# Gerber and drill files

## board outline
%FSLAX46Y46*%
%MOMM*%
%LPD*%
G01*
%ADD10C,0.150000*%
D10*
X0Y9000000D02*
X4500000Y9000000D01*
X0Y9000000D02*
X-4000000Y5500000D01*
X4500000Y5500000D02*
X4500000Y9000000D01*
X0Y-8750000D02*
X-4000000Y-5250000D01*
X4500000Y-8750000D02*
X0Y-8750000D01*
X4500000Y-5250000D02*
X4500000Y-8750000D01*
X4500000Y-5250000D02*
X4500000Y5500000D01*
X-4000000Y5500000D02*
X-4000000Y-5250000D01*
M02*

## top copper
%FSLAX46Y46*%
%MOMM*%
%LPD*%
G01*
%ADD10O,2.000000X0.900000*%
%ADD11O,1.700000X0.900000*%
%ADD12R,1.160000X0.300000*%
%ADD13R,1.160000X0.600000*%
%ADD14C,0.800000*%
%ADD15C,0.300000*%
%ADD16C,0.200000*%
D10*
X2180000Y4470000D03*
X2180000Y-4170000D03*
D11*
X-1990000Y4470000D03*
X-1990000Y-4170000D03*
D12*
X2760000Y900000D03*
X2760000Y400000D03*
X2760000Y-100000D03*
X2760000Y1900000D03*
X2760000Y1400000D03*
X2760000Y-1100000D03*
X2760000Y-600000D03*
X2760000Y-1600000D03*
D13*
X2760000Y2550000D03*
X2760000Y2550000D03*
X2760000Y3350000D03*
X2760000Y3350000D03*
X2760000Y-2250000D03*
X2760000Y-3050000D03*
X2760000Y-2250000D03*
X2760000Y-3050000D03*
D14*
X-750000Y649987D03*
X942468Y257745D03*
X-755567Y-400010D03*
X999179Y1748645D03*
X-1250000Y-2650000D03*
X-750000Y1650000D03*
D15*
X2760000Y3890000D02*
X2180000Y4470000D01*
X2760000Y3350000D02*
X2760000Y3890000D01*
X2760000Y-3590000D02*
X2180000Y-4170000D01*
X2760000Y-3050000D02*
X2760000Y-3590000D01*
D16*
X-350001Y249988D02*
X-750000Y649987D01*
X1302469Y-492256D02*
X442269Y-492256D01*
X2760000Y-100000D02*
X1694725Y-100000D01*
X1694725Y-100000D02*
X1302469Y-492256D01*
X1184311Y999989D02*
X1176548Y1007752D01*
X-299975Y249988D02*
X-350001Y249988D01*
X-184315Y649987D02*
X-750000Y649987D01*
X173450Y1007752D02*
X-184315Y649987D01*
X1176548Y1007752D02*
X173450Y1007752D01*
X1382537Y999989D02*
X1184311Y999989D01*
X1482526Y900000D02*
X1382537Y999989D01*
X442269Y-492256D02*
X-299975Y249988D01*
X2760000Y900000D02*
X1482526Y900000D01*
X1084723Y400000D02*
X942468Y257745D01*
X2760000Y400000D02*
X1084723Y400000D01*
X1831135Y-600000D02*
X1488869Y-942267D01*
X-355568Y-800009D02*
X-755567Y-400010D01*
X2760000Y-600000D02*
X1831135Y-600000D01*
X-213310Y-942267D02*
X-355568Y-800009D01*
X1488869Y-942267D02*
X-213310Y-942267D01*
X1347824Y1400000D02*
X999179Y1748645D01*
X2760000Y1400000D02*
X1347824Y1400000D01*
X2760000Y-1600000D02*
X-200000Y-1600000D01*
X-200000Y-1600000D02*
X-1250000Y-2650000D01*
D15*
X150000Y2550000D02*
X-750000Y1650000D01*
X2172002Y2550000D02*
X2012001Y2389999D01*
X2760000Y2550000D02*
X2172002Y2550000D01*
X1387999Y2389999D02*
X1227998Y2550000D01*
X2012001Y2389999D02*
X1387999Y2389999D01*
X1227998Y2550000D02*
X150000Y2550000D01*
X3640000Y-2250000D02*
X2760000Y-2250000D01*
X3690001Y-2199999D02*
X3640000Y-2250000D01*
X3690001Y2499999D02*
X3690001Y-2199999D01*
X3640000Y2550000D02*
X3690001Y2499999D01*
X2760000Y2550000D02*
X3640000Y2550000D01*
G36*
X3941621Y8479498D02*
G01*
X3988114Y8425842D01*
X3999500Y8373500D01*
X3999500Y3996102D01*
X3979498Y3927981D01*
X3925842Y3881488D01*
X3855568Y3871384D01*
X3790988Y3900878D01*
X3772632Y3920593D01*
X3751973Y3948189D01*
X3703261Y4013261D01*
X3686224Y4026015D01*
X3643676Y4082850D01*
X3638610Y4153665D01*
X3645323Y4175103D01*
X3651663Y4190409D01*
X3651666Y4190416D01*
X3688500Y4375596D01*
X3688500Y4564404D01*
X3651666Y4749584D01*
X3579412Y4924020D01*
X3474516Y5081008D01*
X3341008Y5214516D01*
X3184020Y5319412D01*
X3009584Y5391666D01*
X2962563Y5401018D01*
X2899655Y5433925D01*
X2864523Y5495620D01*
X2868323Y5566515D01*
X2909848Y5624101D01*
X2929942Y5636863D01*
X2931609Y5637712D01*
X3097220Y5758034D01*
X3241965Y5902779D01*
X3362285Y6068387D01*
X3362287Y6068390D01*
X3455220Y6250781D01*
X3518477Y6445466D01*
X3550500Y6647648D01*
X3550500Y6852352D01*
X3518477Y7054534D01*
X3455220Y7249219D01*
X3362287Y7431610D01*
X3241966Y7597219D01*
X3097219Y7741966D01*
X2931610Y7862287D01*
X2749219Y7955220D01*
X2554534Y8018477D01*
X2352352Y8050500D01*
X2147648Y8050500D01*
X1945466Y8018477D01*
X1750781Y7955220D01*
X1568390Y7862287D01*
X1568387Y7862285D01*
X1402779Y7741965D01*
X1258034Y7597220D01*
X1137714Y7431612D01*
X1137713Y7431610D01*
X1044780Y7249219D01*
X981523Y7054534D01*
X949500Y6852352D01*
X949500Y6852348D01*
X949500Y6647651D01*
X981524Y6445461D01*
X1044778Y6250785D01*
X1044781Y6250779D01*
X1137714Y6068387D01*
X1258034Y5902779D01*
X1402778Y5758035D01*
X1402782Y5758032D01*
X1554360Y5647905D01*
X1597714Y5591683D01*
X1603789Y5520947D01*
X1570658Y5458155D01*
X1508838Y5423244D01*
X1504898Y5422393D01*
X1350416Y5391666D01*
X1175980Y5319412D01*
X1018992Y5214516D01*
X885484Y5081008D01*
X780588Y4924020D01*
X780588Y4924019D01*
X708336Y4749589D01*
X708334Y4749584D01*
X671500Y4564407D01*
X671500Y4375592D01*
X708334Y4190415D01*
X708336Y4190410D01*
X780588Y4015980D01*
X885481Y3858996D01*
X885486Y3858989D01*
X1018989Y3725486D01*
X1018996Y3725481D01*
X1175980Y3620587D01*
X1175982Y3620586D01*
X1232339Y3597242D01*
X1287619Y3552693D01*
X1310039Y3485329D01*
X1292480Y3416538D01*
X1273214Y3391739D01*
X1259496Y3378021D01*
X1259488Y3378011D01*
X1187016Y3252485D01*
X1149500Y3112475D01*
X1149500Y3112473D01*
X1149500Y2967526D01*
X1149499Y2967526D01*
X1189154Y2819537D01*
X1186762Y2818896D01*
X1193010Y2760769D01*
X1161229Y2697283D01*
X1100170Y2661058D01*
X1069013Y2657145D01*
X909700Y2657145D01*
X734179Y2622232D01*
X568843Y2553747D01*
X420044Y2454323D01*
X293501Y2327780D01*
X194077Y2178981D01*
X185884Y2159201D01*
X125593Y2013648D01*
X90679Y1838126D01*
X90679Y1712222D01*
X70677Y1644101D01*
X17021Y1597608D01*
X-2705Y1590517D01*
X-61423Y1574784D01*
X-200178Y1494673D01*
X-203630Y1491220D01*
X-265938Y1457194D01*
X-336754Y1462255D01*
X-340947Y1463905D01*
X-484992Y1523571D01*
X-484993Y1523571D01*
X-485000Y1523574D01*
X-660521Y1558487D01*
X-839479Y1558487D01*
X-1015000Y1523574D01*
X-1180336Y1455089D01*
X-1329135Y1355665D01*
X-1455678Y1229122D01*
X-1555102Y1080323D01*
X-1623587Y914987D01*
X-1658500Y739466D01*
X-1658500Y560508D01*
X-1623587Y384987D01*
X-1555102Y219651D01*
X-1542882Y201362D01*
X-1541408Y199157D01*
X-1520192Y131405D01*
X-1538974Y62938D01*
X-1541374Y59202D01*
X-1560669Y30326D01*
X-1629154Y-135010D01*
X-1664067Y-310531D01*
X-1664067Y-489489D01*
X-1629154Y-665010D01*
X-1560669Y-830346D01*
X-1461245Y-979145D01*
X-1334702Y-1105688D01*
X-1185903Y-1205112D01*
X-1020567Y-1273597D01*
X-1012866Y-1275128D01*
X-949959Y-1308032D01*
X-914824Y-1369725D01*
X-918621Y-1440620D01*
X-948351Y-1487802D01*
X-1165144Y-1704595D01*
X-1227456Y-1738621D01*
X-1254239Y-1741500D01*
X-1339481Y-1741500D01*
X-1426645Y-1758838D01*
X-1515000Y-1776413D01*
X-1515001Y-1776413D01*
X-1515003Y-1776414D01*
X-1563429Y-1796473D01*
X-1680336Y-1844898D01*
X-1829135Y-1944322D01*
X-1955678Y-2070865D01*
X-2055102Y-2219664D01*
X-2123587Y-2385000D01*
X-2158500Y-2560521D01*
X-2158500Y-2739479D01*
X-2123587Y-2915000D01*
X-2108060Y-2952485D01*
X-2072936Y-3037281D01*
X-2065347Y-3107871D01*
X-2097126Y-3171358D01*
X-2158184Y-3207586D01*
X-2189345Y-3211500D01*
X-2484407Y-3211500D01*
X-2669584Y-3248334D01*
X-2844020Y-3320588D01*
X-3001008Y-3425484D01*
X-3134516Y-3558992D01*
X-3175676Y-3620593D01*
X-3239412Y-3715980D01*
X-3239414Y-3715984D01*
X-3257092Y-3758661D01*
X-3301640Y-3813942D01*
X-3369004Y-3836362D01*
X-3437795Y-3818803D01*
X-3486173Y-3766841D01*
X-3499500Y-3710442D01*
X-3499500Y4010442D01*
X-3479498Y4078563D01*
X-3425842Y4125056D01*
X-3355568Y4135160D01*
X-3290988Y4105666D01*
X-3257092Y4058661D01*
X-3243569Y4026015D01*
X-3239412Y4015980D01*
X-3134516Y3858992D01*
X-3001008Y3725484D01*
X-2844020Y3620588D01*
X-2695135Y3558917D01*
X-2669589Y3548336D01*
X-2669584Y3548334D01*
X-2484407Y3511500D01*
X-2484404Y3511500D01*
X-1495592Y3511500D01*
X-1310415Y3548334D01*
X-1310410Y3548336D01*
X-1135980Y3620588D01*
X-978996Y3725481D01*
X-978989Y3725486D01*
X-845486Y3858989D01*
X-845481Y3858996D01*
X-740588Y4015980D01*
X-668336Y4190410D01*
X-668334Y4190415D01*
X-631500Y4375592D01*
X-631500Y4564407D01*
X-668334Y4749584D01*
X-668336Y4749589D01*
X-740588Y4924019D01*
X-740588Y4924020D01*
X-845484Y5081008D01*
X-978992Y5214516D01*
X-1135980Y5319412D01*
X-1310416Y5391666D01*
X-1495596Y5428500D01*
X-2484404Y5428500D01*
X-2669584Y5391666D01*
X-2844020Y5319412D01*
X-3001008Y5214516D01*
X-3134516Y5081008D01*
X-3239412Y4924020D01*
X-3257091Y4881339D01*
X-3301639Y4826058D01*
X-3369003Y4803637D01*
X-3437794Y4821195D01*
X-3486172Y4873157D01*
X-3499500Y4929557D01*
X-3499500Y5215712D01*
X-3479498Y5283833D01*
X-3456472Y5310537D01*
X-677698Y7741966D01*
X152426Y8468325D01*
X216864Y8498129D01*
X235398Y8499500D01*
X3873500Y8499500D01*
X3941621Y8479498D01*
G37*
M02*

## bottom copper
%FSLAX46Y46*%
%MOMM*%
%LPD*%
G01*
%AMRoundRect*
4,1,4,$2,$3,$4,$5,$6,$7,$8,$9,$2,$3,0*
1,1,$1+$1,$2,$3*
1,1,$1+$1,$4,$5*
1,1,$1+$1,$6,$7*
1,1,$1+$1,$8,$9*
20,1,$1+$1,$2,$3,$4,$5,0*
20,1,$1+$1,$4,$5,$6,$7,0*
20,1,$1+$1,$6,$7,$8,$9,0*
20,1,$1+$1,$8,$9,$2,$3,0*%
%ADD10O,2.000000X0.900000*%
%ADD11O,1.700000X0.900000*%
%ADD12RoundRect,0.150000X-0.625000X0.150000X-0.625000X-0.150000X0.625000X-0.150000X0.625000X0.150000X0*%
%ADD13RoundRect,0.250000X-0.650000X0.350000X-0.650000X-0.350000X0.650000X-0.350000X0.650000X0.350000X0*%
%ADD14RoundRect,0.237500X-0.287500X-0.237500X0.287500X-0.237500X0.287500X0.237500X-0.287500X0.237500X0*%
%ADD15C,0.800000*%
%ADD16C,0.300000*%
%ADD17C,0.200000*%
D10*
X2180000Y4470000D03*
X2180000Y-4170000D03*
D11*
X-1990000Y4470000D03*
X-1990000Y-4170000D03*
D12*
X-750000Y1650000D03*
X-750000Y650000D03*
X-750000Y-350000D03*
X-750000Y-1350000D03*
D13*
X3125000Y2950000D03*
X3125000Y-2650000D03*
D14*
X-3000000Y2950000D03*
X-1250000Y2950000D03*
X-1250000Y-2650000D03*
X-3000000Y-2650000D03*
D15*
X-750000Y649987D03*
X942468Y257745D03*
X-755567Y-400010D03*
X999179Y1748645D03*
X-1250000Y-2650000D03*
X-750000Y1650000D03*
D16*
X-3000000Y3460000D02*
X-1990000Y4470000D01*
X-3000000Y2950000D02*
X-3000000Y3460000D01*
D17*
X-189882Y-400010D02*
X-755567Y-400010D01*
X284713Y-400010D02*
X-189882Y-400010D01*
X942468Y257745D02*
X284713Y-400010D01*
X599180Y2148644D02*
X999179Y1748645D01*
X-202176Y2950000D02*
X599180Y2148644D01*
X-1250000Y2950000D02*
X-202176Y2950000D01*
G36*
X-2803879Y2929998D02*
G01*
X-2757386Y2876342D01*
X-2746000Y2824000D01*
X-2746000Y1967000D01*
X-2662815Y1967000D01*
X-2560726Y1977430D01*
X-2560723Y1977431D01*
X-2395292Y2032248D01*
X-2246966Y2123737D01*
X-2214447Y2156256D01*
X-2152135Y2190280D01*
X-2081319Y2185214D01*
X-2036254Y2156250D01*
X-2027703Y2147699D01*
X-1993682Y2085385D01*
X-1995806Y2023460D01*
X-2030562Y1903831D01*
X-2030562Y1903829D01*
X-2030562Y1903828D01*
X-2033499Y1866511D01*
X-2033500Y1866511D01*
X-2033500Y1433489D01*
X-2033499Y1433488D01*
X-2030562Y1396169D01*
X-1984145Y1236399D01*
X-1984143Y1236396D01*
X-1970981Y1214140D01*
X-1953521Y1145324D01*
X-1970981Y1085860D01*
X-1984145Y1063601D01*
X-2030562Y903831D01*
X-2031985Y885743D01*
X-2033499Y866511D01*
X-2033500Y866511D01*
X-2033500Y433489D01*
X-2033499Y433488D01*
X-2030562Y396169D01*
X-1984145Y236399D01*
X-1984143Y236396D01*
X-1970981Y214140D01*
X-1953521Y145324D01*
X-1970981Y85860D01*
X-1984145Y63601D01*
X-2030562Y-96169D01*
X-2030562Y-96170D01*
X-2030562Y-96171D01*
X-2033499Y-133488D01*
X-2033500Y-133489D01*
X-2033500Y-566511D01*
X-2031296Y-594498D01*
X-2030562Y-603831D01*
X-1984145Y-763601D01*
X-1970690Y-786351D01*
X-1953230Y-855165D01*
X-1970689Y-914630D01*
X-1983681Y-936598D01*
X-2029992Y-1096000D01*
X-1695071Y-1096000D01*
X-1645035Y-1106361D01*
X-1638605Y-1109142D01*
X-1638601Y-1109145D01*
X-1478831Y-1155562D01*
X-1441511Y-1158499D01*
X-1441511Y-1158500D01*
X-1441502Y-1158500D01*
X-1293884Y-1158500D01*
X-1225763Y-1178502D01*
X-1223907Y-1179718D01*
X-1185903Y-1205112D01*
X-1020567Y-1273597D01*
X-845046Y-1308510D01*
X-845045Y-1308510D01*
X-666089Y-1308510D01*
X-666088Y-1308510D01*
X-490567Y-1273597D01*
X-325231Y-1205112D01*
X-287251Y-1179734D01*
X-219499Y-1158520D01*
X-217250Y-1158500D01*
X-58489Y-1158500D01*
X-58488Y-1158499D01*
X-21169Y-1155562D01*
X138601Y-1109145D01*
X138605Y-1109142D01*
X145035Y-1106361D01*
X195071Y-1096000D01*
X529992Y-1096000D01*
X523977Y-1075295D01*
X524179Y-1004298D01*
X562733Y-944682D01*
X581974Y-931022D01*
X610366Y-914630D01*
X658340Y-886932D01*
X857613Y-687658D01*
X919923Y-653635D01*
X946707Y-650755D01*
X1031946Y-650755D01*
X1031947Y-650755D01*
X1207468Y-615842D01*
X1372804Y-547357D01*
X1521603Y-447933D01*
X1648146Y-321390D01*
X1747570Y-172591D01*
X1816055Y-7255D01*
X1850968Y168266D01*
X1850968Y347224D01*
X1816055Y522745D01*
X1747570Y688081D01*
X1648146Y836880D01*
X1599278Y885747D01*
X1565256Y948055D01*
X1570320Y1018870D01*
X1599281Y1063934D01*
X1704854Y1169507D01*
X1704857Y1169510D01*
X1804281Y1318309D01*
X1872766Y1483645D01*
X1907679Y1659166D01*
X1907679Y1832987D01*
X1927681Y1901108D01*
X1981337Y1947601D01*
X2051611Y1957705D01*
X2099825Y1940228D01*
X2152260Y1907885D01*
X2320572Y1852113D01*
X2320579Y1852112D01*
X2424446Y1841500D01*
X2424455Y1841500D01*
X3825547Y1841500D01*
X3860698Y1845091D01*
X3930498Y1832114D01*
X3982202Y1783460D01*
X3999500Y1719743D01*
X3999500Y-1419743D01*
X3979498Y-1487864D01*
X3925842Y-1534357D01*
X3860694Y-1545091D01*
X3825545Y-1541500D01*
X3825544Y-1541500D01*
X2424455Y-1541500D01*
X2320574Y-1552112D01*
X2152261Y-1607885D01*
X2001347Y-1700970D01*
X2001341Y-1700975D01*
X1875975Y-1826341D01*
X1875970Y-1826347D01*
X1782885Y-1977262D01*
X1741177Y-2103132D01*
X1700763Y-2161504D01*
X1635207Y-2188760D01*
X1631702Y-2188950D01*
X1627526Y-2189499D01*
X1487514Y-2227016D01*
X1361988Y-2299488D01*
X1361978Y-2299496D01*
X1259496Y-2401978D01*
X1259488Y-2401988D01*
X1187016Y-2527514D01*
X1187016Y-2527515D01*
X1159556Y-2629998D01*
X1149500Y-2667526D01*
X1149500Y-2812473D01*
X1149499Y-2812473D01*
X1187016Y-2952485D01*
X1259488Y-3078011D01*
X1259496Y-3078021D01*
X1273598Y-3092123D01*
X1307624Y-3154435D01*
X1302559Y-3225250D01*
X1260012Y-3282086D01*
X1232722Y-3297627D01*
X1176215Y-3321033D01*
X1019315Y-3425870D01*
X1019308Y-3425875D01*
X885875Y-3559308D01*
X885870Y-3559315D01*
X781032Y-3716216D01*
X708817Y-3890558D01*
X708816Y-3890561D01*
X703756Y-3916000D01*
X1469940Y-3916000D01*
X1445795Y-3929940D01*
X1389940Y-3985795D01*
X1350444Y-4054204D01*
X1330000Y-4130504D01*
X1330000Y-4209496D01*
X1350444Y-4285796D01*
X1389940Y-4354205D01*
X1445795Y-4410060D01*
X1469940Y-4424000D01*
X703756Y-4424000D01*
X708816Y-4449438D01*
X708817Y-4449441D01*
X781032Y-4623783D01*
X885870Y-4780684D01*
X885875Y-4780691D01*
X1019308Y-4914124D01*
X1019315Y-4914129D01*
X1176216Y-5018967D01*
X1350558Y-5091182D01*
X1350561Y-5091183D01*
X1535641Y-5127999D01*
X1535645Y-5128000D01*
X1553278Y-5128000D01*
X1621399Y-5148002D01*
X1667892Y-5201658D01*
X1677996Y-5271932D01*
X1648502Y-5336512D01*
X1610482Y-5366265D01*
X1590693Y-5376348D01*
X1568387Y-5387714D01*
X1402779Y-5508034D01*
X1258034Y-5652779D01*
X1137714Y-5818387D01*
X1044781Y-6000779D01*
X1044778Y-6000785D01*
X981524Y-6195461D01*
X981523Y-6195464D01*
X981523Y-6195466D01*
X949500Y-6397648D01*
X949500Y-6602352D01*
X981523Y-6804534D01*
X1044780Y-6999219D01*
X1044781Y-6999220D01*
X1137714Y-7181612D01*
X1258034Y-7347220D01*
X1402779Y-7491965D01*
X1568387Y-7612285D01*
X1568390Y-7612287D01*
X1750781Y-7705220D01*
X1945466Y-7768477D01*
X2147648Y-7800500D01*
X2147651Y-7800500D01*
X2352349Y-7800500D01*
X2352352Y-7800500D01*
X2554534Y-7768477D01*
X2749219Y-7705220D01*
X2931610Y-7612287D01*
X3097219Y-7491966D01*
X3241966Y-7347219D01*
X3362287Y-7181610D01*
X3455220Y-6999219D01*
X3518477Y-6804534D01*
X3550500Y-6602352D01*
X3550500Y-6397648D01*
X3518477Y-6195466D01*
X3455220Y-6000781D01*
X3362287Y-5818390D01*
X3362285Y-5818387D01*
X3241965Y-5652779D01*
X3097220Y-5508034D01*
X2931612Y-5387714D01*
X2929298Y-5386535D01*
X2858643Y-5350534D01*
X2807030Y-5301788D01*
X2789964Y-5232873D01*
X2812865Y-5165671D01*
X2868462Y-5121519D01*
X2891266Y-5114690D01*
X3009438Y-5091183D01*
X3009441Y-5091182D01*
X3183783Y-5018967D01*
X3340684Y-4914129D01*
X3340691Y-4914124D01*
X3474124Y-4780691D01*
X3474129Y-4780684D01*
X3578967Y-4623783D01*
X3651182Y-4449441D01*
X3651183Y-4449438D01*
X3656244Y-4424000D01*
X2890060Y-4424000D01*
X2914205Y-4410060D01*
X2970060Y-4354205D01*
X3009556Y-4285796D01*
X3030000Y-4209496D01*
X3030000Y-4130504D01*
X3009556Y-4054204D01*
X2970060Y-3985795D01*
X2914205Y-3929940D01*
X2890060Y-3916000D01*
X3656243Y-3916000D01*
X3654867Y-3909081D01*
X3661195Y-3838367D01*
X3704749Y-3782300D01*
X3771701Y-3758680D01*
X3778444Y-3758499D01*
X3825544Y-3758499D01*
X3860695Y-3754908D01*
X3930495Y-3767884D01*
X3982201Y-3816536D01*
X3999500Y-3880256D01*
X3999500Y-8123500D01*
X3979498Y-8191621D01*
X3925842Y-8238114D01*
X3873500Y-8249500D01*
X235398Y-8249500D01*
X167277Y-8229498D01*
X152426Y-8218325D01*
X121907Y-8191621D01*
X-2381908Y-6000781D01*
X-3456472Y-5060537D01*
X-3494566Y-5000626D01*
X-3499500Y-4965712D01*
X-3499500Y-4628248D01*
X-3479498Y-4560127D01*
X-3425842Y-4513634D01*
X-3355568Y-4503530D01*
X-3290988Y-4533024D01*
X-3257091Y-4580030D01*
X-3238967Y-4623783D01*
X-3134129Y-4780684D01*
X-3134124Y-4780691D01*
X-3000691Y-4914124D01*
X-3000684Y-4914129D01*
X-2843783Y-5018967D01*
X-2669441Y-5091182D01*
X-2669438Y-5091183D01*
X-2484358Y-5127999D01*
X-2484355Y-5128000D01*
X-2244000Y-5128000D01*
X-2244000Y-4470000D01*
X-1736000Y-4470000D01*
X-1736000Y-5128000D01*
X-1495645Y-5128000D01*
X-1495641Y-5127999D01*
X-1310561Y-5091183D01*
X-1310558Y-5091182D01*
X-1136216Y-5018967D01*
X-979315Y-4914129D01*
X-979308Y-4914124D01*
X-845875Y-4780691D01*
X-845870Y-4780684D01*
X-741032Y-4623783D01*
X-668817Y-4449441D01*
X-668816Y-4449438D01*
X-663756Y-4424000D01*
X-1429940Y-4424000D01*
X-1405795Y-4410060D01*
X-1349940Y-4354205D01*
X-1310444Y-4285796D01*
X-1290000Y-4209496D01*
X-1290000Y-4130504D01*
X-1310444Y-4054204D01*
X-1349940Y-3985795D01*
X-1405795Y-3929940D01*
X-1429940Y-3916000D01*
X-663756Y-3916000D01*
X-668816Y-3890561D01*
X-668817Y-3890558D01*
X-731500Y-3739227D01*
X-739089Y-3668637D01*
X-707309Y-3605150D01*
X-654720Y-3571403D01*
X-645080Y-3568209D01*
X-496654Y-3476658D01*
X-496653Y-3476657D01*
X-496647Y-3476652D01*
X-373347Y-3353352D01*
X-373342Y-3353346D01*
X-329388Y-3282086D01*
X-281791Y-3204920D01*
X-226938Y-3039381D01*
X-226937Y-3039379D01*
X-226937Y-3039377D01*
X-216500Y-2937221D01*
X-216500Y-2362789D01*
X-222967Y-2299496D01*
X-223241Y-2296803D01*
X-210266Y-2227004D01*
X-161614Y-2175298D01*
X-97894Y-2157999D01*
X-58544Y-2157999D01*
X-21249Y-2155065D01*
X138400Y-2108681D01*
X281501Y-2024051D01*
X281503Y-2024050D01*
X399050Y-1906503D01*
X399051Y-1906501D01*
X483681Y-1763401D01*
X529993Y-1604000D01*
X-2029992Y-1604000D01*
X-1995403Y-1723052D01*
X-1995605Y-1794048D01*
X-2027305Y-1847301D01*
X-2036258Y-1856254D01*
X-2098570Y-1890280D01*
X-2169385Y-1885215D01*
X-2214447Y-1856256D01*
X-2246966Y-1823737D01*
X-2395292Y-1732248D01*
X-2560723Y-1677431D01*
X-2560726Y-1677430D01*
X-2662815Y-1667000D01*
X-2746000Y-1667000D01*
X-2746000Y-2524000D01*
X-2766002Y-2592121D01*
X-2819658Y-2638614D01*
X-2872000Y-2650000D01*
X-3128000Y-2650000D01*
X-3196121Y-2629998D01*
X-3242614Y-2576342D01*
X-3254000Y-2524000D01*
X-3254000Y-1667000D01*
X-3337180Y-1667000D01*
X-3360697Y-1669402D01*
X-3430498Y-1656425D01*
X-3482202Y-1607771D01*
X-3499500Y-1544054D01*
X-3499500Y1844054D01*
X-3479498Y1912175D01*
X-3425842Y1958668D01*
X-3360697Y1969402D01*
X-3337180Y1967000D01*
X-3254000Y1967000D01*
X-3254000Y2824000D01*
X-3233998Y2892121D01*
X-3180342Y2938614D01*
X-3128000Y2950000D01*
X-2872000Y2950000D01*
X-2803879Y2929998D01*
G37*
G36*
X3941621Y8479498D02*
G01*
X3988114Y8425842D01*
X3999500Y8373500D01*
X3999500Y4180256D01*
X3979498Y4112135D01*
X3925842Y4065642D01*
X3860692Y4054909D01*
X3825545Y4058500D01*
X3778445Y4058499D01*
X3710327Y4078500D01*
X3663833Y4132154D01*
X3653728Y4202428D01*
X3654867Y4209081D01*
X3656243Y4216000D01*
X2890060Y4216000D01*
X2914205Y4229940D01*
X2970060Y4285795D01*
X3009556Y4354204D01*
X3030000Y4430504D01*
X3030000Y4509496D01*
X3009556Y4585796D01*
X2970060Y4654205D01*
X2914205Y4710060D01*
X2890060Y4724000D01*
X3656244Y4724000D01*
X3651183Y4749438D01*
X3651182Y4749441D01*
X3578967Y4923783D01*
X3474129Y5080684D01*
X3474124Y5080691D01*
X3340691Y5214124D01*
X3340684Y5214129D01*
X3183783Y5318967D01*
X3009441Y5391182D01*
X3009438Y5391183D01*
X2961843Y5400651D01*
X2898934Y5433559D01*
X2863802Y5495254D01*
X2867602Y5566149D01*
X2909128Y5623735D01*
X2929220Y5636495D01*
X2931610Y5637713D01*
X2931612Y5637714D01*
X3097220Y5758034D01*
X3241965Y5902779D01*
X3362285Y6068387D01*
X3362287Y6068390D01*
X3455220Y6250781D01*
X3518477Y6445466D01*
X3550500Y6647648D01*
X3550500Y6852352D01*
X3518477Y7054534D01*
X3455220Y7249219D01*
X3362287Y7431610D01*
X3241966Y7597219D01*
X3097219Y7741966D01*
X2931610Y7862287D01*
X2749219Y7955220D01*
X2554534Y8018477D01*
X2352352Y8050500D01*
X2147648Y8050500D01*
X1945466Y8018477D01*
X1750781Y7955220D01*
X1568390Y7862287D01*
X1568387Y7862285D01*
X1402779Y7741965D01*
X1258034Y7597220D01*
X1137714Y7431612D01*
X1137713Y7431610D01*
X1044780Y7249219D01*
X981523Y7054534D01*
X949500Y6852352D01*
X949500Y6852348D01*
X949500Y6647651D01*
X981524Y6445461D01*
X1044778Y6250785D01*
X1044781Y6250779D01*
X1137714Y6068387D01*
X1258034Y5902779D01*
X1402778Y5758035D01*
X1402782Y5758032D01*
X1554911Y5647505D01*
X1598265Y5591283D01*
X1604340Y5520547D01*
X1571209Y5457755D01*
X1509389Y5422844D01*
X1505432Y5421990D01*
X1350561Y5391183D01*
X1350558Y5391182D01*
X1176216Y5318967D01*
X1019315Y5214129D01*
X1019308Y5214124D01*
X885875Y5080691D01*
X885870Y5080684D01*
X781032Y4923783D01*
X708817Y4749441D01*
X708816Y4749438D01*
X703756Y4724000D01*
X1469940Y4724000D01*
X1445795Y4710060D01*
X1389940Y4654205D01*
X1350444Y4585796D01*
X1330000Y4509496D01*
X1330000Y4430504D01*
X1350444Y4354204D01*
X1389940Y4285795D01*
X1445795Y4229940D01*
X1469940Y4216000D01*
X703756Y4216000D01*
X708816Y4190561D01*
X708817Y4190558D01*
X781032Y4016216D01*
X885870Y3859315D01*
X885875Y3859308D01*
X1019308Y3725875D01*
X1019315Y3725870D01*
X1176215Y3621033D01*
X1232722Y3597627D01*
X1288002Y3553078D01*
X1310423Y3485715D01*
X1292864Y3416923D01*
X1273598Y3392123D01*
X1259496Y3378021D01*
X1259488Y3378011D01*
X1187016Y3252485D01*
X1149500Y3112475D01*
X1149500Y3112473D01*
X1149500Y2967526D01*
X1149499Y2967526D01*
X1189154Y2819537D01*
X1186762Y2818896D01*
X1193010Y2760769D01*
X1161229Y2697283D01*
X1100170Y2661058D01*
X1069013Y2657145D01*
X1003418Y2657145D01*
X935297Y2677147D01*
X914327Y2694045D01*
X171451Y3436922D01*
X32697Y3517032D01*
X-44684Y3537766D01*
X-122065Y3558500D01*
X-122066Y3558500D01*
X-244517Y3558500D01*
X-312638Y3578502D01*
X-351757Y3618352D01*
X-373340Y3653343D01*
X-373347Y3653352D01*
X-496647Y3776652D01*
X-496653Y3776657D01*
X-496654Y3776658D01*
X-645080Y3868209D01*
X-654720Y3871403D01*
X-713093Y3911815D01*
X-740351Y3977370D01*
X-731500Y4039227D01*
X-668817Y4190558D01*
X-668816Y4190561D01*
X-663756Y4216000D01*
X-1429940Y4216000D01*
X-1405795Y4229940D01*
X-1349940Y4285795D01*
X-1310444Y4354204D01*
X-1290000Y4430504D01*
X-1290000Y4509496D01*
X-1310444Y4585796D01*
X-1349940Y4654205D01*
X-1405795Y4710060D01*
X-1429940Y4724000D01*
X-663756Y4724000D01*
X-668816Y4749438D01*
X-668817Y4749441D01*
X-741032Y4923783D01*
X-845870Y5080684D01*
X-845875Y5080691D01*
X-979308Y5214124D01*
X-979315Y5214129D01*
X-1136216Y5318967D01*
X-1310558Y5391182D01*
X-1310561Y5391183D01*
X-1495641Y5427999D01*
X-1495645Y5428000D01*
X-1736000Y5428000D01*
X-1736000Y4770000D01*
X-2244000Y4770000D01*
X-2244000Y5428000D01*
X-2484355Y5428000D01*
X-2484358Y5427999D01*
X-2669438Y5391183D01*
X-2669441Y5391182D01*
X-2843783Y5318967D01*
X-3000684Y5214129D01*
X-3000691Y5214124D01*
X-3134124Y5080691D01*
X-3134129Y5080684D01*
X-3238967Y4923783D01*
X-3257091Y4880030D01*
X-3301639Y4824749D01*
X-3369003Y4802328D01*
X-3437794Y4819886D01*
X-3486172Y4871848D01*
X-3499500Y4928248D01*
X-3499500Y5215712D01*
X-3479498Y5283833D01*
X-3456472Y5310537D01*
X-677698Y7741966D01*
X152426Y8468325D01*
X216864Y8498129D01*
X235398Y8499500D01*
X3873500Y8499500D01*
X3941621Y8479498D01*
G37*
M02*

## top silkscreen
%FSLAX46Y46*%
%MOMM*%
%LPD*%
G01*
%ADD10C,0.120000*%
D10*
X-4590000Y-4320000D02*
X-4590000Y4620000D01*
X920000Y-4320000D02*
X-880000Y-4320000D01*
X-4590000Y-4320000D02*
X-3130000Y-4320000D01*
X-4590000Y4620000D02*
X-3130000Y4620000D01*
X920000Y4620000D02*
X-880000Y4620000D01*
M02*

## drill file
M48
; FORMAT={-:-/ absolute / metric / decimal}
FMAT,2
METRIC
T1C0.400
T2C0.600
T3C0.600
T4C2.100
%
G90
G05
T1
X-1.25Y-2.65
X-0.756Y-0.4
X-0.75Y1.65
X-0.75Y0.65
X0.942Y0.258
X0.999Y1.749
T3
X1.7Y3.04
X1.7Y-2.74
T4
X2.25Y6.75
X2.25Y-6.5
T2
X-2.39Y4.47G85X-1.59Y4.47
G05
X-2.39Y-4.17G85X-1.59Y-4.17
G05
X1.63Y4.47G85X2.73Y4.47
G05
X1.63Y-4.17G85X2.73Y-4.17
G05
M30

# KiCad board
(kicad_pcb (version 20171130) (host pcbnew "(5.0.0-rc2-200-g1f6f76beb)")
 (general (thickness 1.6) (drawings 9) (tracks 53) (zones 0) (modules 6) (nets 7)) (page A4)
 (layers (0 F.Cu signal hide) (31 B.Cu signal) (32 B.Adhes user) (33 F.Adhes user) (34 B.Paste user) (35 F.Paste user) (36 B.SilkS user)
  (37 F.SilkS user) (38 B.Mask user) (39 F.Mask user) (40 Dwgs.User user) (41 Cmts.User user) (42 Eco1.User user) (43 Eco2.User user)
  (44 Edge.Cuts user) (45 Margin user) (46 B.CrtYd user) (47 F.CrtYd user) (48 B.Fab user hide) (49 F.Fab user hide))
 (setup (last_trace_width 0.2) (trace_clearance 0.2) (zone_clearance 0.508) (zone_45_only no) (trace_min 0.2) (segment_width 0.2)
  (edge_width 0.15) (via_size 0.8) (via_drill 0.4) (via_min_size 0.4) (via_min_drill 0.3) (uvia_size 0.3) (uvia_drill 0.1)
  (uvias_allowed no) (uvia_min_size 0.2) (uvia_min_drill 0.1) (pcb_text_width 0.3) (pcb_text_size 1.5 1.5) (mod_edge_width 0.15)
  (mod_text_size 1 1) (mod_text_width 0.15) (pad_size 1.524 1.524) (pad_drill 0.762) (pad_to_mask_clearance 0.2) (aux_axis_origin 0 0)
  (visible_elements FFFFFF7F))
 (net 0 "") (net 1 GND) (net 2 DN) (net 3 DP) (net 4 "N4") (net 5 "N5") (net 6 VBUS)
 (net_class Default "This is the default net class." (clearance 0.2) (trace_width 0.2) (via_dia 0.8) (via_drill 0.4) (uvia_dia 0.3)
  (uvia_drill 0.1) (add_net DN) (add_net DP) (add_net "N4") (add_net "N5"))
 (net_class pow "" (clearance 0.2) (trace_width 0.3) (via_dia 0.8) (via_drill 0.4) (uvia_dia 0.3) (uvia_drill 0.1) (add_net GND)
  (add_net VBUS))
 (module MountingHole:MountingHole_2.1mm (layer F.Cu) (at 2.25 -6.75)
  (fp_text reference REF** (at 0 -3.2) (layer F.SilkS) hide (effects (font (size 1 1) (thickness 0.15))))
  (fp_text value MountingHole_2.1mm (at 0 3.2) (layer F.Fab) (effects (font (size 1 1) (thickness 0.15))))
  (pad "" np_thru_hole circle (at 0 0) (size 2.1 2.1) (drill 2.1) (layers *.Cu *.Mask)))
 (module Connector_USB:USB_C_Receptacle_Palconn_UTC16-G (layer F.Cu) (at 0.25 -0.15 270)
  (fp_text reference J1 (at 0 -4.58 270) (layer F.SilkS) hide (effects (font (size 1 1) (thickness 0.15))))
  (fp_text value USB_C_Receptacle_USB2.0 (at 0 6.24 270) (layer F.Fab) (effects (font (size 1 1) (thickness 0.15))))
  (fp_line (start 4.47 4.84) (end -4.47 4.84) (layer F.SilkS) (width 0.12))
  (fp_line (start 4.47 -0.67) (end 4.47 1.13) (layer F.SilkS) (width 0.12))
  (fp_line (start 4.47 4.84) (end 4.47 3.38) (layer F.SilkS) (width 0.12))
  (fp_line (start -4.47 4.84) (end -4.47 3.38) (layer F.SilkS) (width 0.12))
  (fp_line (start -4.47 -0.67) (end -4.47 1.13) (layer F.SilkS) (width 0.12))
  (pad S1 thru_hole oval (at -4.32 -1.93) (size 2 0.9) (drill oval 1.7 0.6) (layers *.Cu *.Mask) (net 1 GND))
  (pad S1 thru_hole oval (at 4.32 -1.93) (size 2 0.9) (drill oval 1.7 0.6) (layers *.Cu *.Mask) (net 1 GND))
  (pad S1 thru_hole oval (at -4.32 2.24) (size 1.7 0.9) (drill oval 1.4 0.6) (layers *.Cu *.Mask) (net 1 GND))
  (pad S1 thru_hole oval (at 4.32 2.24) (size 1.7 0.9) (drill oval 1.4 0.6) (layers *.Cu *.Mask) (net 1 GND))
  (pad B7 smd rect (at -0.75 -2.51 90) (size 0.3 1.16) (layers F.Cu F.Paste F.Mask) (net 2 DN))
  (pad A6 smd rect (at -0.25 -2.51 90) (size 0.3 1.16) (layers F.Cu F.Paste F.Mask) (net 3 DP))
  (pad A7 smd rect (at 0.25 -2.51 90) (size 0.3 1.16) (layers F.Cu F.Paste F.Mask) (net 2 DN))
  (pad B8 smd rect (at -1.75 -2.51 90) (size 0.3 1.16) (layers F.Cu F.Paste F.Mask))
  (pad A5 smd rect (at -1.25 -2.51 90) (size 0.3 1.16) (layers F.Cu F.Paste F.Mask) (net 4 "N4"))
  (pad A8 smd rect (at 1.25 -2.51 90) (size 0.3 1.16) (layers F.Cu F.Paste F.Mask))
  (pad B6 smd rect (at 0.75 -2.51 90) (size 0.3 1.16) (layers F.Cu F.Paste F.Mask) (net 3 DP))
  (pad B5 smd rect (at 1.75 -2.51 90) (size 0.3 1.16) (layers F.Cu F.Paste F.Mask) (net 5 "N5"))
  (pad "" np_thru_hole circle (at 2.89 -1.45 90) (size 0.6 0.6) (drill 0.6) (layers *.Cu *.Mask))
  (pad "" np_thru_hole circle (at -2.89 -1.45 90) (size 0.6 0.6) (drill 0.6) (layers *.Cu *.Mask))
  (pad A4 smd rect (at -2.4 -2.51 270) (size 0.6 1.16) (layers F.Cu F.Paste F.Mask) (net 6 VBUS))
  (pad B9 smd rect (at -2.4 -2.51 270) (size 0.6 1.16) (layers F.Cu F.Paste F.Mask) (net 6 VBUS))
  (pad A1 smd rect (at -3.2 -2.51 270) (size 0.6 1.16) (layers F.Cu F.Paste F.Mask) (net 1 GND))
  (pad B12 smd rect (at -3.2 -2.51 270) (size 0.6 1.16) (layers F.Cu F.Paste F.Mask) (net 1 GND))
  (pad B4 smd rect (at 2.4 -2.51 270) (size 0.6 1.16) (layers F.Cu F.Paste F.Mask) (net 6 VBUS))
  (pad B1 smd rect (at 3.2 -2.51 270) (size 0.6 1.16) (layers F.Cu F.Paste F.Mask) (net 1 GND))
  (pad A9 smd rect (at 2.4 -2.51 270) (size 0.6 1.16) (layers F.Cu F.Paste F.Mask) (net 6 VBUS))
  (pad A12 smd rect (at 3.2 -2.51 270) (size 0.6 1.16) (layers F.Cu F.Paste F.Mask) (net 1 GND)))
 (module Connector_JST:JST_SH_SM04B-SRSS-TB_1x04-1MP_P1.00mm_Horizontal (layer B.Cu) (at 1.25 -0.15 270)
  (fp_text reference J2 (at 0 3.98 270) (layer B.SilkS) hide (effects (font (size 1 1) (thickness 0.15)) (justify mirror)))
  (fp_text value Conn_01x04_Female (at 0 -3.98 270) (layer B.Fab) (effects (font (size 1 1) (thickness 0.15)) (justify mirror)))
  (pad 1 smd roundrect (at -1.5 2 270) (size 0.6 1.55) (layers B.Cu B.Paste B.Mask) (roundrect_rratio 0.25) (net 6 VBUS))
  (pad 2 smd roundrect (at -0.5 2 270) (size 0.6 1.55) (layers B.Cu B.Paste B.Mask) (roundrect_rratio 0.25) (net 2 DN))
  (pad 3 smd roundrect (at 0.5 2 270) (size 0.6 1.55) (layers B.Cu B.Paste B.Mask) (roundrect_rratio 0.25) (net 3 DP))
  (pad 4 smd roundrect (at 1.5 2 270) (size 0.6 1.55) (layers B.Cu B.Paste B.Mask) (roundrect_rratio 0.25) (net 1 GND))
  (pad MP smd roundrect (at -2.8 -1.875 270) (size 1.2 1.8) (layers B.Cu B.Paste B.Mask) (roundrect_rratio 0.208333))
  (pad MP smd roundrect (at 2.8 -1.875 270) (size 1.2 1.8) (layers B.Cu B.Paste B.Mask) (roundrect_rratio 0.208333)))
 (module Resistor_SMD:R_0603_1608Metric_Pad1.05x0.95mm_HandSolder (layer B.Cu) (at -2.125 -2.95)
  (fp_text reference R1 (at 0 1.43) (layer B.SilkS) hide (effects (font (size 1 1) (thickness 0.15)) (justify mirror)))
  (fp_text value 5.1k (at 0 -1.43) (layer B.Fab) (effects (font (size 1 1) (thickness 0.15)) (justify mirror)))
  (pad 1 smd roundrect (at -0.875 0) (size 1.05 0.95) (layers B.Cu B.Paste B.Mask) (roundrect_rratio 0.25) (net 1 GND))
  (pad 2 smd roundrect (at 0.875 0) (size 1.05 0.95) (layers B.Cu B.Paste B.Mask) (roundrect_rratio 0.25) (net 4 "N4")))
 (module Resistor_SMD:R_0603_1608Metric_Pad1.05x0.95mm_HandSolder (layer B.Cu) (at -2.125 2.65)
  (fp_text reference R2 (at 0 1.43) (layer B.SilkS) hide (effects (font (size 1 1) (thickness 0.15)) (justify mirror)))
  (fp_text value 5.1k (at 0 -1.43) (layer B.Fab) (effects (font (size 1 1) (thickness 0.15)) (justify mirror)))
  (pad 2 smd roundrect (at 0.875 0) (size 1.05 0.95) (layers B.Cu B.Paste B.Mask) (roundrect_rratio 0.25) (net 5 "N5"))
  (pad 1 smd roundrect (at -0.875 0) (size 1.05 0.95) (layers B.Cu B.Paste B.Mask) (roundrect_rratio 0.25) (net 1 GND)))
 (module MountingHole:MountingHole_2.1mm (layer F.Cu) (at 2.25 6.5)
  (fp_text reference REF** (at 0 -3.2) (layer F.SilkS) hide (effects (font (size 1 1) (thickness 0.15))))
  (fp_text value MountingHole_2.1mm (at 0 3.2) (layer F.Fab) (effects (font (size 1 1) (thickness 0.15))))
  (pad "" np_thru_hole circle (at 0 0) (size 2.1 2.1) (drill 2.1) (layers *.Cu *.Mask)))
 (gr_line (start 0 -9) (end 4.5 -9) (layer Edge.Cuts) (width 0.15))
 (gr_line (start 0 -9) (end -4 -5.5) (layer Edge.Cuts) (width 0.15))
 (gr_line (start 4.5 -5.5) (end 4.5 -9) (layer Edge.Cuts) (width 0.15))
 (gr_line (start 0 8.75) (end -4 5.25) (layer Edge.Cuts) (width 0.15))
 (gr_line (start 4.5 8.75) (end 0 8.75) (layer Edge.Cuts) (width 0.15))
 (gr_line (start 4.5 5.25) (end 4.5 8.75) (layer Edge.Cuts) (width 0.15))
 (gr_line (start 4.5 5.25) (end 4.5 -5.5) (layer Edge.Cuts) (width 0.15))
 (gr_line (start -4 -5.5) (end -4 5.25) (layer Edge.Cuts) (width 0.15))
 (segment (start 2.76 -3.89) (end 2.18 -4.47) (width 0.3) (layer F.Cu) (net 1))
 (segment (start 2.76 -3.35) (end 2.76 -3.89) (width 0.3) (layer F.Cu) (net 1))
 (segment (start 2.76 3.59) (end 2.18 4.17) (width 0.3) (layer F.Cu) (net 1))
 (segment (start 2.76 3.05) (end 2.76 3.59) (width 0.3) (layer F.Cu) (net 1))
 (segment (start -3 -3.46) (end -1.99 -4.47) (width 0.3) (layer B.Cu) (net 1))
 (segment (start -3 -2.95) (end -3 -3.46) (width 0.3) (layer B.Cu) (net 1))
 (via (at -0.75 -0.649987) (size 0.8) (drill 0.4) (layers F.Cu B.Cu) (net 2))
 (segment (start -0.350001 -0.249988) (end -0.75 -0.649987) (width 0.2) (layer F.Cu) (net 2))
 (segment (start 1.302469 0.492256) (end 0.442269 0.492256) (width 0.2) (layer F.Cu) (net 2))
 (segment (start 2.76 0.1) (end 1.694725 0.1) (width 0.2) (layer F.Cu) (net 2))
 (segment (start 1.694725 0.1) (end 1.302469 0.492256) (width 0.2) (layer F.Cu) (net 2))
 (segment (start 1.184311 -0.999989) (end 1.176548 -1.007752) (width 0.2) (layer F.Cu) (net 2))
 (segment (start -0.299975 -0.249988) (end -0.350001 -0.249988) (width 0.2) (layer F.Cu) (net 2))
 (segment (start -0.184315 -0.649987) (end -0.75 -0.649987) (width 0.2) (layer F.Cu) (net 2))
 (segment (start 0.17345 -1.007752) (end -0.184315 -0.649987) (width 0.2) (layer F.Cu) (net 2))
 (segment (start 1.176548 -1.007752) (end 0.17345 -1.007752) (width 0.2) (layer F.Cu) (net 2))
 (segment (start 1.382537 -0.999989) (end 1.184311 -0.999989) (width 0.2) (layer F.Cu) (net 2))
 (segment (start 1.482526 -0.9) (end 1.382537 -0.999989) (width 0.2) (layer F.Cu) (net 2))
 (segment (start 0.442269 0.492256) (end -0.299975 -0.249988) (width 0.2) (layer F.Cu) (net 2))
 (segment (start 2.76 -0.9) (end 1.482526 -0.9) (width 0.2) (layer F.Cu) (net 2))
 (via (at 0.942468 -0.257745) (size 0.8) (drill 0.4) (layers F.Cu B.Cu) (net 3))
 (segment (start 1.084723 -0.4) (end 0.942468 -0.257745) (width 0.2) (layer F.Cu) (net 3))
 (segment (start 2.76 -0.4) (end 1.084723 -0.4) (width 0.2) (layer F.Cu) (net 3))
 (segment (start 1.831135 0.6) (end 1.488869 0.942267) (width 0.2) (layer F.Cu) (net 3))
 (segment (start -0.355568 0.800009) (end -0.755567 0.40001) (width 0.2) (layer F.Cu) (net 3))
 (segment (start -0.189882 0.40001) (end -0.755567 0.40001) (width 0.2) (layer B.Cu) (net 3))
 (segment (start 2.76 0.6) (end 1.831135 0.6) (width 0.2) (layer F.Cu) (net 3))
 (segment (start -0.21331 0.942267) (end -0.355568 0.800009) (width 0.2) (layer F.Cu) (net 3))
 (segment (start 0.284713 0.40001) (end -0.189882 0.40001) (width 0.2) (layer B.Cu) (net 3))
 (segment (start 0.942468 -0.257745) (end 0.284713 0.40001) (width 0.2) (layer B.Cu) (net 3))
 (segment (start 1.488869 0.942267) (end -0.21331 0.942267) (width 0.2) (layer F.Cu) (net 3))
 (via (at -0.755567 0.40001) (size 0.8) (drill 0.4) (layers F.Cu B.Cu) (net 3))
 (segment (start 0.59918 -2.148644) (end 0.999179 -1.748645) (width 0.2) (layer B.Cu) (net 4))
 (segment (start -0.202176 -2.95) (end 0.59918 -2.148644) (width 0.2) (layer B.Cu) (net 4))
 (segment (start -1.25 -2.95) (end -0.202176 -2.95) (width 0.2) (layer B.Cu) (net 4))
 (segment (start 1.347824 -1.4) (end 0.999179 -1.748645) (width 0.2) (layer F.Cu) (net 4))
 (segment (start 2.76 -1.4) (end 1.347824 -1.4) (width 0.2) (layer F.Cu) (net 4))
 (via (at 0.999179 -1.748645) (size 0.8) (drill 0.4) (layers F.Cu B.Cu) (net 4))
 (via (at -1.25 2.65) (size 0.8) (drill 0.4) (layers F.Cu B.Cu) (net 5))
 (segment (start 2.76 1.6) (end -0.2 1.6) (width 0.2) (layer F.Cu) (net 5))
 (segment (start -0.2 1.6) (end -1.25 2.65) (width 0.2) (layer F.Cu) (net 5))
 (segment (start 0.15 -2.55) (end -0.75 -1.65) (width 0.3) (layer F.Cu) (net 6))
 (segment (start 2.172002 -2.55) (end 2.012001 -2.389999) (width 0.3) (layer F.Cu) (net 6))
 (segment (start 2.76 -2.55) (end 2.172002 -2.55) (width 0.3) (layer F.Cu) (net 6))
 (segment (start 1.387999 -2.389999) (end 1.227998 -2.55) (width 0.3) (layer F.Cu) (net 6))
 (segment (start 2.012001 -2.389999) (end 1.387999 -2.389999) (width 0.3) (layer F.Cu) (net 6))
 (via (at -0.75 -1.65) (size 0.8) (drill 0.4) (layers F.Cu B.Cu) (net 6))
 (segment (start 1.227998 -2.55) (end 0.15 -2.55) (width 0.3) (layer F.Cu) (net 6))
 (segment (start 3.64 2.25) (end 2.76 2.25) (width 0.3) (layer F.Cu) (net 6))
 (segment (start 3.690001 2.199999) (end 3.64 2.25) (width 0.3) (layer F.Cu) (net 6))
 (segment (start 3.690001 -2.499999) (end 3.690001 2.199999) (width 0.3) (layer F.Cu) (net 6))
 (segment (start 3.64 -2.55) (end 3.690001 -2.499999) (width 0.3) (layer F.Cu) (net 6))
 (segment (start 2.76 -2.55) (end 3.64 -2.55) (width 0.3) (layer F.Cu) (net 6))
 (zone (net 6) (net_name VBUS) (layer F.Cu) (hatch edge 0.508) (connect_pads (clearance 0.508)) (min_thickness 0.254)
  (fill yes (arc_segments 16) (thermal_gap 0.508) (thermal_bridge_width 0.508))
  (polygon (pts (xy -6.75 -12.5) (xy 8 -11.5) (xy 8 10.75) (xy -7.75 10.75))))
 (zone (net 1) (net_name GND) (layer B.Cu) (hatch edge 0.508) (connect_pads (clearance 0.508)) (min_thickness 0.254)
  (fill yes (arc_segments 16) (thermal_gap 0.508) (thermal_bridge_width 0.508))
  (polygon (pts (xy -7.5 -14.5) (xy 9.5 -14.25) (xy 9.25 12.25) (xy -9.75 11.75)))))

